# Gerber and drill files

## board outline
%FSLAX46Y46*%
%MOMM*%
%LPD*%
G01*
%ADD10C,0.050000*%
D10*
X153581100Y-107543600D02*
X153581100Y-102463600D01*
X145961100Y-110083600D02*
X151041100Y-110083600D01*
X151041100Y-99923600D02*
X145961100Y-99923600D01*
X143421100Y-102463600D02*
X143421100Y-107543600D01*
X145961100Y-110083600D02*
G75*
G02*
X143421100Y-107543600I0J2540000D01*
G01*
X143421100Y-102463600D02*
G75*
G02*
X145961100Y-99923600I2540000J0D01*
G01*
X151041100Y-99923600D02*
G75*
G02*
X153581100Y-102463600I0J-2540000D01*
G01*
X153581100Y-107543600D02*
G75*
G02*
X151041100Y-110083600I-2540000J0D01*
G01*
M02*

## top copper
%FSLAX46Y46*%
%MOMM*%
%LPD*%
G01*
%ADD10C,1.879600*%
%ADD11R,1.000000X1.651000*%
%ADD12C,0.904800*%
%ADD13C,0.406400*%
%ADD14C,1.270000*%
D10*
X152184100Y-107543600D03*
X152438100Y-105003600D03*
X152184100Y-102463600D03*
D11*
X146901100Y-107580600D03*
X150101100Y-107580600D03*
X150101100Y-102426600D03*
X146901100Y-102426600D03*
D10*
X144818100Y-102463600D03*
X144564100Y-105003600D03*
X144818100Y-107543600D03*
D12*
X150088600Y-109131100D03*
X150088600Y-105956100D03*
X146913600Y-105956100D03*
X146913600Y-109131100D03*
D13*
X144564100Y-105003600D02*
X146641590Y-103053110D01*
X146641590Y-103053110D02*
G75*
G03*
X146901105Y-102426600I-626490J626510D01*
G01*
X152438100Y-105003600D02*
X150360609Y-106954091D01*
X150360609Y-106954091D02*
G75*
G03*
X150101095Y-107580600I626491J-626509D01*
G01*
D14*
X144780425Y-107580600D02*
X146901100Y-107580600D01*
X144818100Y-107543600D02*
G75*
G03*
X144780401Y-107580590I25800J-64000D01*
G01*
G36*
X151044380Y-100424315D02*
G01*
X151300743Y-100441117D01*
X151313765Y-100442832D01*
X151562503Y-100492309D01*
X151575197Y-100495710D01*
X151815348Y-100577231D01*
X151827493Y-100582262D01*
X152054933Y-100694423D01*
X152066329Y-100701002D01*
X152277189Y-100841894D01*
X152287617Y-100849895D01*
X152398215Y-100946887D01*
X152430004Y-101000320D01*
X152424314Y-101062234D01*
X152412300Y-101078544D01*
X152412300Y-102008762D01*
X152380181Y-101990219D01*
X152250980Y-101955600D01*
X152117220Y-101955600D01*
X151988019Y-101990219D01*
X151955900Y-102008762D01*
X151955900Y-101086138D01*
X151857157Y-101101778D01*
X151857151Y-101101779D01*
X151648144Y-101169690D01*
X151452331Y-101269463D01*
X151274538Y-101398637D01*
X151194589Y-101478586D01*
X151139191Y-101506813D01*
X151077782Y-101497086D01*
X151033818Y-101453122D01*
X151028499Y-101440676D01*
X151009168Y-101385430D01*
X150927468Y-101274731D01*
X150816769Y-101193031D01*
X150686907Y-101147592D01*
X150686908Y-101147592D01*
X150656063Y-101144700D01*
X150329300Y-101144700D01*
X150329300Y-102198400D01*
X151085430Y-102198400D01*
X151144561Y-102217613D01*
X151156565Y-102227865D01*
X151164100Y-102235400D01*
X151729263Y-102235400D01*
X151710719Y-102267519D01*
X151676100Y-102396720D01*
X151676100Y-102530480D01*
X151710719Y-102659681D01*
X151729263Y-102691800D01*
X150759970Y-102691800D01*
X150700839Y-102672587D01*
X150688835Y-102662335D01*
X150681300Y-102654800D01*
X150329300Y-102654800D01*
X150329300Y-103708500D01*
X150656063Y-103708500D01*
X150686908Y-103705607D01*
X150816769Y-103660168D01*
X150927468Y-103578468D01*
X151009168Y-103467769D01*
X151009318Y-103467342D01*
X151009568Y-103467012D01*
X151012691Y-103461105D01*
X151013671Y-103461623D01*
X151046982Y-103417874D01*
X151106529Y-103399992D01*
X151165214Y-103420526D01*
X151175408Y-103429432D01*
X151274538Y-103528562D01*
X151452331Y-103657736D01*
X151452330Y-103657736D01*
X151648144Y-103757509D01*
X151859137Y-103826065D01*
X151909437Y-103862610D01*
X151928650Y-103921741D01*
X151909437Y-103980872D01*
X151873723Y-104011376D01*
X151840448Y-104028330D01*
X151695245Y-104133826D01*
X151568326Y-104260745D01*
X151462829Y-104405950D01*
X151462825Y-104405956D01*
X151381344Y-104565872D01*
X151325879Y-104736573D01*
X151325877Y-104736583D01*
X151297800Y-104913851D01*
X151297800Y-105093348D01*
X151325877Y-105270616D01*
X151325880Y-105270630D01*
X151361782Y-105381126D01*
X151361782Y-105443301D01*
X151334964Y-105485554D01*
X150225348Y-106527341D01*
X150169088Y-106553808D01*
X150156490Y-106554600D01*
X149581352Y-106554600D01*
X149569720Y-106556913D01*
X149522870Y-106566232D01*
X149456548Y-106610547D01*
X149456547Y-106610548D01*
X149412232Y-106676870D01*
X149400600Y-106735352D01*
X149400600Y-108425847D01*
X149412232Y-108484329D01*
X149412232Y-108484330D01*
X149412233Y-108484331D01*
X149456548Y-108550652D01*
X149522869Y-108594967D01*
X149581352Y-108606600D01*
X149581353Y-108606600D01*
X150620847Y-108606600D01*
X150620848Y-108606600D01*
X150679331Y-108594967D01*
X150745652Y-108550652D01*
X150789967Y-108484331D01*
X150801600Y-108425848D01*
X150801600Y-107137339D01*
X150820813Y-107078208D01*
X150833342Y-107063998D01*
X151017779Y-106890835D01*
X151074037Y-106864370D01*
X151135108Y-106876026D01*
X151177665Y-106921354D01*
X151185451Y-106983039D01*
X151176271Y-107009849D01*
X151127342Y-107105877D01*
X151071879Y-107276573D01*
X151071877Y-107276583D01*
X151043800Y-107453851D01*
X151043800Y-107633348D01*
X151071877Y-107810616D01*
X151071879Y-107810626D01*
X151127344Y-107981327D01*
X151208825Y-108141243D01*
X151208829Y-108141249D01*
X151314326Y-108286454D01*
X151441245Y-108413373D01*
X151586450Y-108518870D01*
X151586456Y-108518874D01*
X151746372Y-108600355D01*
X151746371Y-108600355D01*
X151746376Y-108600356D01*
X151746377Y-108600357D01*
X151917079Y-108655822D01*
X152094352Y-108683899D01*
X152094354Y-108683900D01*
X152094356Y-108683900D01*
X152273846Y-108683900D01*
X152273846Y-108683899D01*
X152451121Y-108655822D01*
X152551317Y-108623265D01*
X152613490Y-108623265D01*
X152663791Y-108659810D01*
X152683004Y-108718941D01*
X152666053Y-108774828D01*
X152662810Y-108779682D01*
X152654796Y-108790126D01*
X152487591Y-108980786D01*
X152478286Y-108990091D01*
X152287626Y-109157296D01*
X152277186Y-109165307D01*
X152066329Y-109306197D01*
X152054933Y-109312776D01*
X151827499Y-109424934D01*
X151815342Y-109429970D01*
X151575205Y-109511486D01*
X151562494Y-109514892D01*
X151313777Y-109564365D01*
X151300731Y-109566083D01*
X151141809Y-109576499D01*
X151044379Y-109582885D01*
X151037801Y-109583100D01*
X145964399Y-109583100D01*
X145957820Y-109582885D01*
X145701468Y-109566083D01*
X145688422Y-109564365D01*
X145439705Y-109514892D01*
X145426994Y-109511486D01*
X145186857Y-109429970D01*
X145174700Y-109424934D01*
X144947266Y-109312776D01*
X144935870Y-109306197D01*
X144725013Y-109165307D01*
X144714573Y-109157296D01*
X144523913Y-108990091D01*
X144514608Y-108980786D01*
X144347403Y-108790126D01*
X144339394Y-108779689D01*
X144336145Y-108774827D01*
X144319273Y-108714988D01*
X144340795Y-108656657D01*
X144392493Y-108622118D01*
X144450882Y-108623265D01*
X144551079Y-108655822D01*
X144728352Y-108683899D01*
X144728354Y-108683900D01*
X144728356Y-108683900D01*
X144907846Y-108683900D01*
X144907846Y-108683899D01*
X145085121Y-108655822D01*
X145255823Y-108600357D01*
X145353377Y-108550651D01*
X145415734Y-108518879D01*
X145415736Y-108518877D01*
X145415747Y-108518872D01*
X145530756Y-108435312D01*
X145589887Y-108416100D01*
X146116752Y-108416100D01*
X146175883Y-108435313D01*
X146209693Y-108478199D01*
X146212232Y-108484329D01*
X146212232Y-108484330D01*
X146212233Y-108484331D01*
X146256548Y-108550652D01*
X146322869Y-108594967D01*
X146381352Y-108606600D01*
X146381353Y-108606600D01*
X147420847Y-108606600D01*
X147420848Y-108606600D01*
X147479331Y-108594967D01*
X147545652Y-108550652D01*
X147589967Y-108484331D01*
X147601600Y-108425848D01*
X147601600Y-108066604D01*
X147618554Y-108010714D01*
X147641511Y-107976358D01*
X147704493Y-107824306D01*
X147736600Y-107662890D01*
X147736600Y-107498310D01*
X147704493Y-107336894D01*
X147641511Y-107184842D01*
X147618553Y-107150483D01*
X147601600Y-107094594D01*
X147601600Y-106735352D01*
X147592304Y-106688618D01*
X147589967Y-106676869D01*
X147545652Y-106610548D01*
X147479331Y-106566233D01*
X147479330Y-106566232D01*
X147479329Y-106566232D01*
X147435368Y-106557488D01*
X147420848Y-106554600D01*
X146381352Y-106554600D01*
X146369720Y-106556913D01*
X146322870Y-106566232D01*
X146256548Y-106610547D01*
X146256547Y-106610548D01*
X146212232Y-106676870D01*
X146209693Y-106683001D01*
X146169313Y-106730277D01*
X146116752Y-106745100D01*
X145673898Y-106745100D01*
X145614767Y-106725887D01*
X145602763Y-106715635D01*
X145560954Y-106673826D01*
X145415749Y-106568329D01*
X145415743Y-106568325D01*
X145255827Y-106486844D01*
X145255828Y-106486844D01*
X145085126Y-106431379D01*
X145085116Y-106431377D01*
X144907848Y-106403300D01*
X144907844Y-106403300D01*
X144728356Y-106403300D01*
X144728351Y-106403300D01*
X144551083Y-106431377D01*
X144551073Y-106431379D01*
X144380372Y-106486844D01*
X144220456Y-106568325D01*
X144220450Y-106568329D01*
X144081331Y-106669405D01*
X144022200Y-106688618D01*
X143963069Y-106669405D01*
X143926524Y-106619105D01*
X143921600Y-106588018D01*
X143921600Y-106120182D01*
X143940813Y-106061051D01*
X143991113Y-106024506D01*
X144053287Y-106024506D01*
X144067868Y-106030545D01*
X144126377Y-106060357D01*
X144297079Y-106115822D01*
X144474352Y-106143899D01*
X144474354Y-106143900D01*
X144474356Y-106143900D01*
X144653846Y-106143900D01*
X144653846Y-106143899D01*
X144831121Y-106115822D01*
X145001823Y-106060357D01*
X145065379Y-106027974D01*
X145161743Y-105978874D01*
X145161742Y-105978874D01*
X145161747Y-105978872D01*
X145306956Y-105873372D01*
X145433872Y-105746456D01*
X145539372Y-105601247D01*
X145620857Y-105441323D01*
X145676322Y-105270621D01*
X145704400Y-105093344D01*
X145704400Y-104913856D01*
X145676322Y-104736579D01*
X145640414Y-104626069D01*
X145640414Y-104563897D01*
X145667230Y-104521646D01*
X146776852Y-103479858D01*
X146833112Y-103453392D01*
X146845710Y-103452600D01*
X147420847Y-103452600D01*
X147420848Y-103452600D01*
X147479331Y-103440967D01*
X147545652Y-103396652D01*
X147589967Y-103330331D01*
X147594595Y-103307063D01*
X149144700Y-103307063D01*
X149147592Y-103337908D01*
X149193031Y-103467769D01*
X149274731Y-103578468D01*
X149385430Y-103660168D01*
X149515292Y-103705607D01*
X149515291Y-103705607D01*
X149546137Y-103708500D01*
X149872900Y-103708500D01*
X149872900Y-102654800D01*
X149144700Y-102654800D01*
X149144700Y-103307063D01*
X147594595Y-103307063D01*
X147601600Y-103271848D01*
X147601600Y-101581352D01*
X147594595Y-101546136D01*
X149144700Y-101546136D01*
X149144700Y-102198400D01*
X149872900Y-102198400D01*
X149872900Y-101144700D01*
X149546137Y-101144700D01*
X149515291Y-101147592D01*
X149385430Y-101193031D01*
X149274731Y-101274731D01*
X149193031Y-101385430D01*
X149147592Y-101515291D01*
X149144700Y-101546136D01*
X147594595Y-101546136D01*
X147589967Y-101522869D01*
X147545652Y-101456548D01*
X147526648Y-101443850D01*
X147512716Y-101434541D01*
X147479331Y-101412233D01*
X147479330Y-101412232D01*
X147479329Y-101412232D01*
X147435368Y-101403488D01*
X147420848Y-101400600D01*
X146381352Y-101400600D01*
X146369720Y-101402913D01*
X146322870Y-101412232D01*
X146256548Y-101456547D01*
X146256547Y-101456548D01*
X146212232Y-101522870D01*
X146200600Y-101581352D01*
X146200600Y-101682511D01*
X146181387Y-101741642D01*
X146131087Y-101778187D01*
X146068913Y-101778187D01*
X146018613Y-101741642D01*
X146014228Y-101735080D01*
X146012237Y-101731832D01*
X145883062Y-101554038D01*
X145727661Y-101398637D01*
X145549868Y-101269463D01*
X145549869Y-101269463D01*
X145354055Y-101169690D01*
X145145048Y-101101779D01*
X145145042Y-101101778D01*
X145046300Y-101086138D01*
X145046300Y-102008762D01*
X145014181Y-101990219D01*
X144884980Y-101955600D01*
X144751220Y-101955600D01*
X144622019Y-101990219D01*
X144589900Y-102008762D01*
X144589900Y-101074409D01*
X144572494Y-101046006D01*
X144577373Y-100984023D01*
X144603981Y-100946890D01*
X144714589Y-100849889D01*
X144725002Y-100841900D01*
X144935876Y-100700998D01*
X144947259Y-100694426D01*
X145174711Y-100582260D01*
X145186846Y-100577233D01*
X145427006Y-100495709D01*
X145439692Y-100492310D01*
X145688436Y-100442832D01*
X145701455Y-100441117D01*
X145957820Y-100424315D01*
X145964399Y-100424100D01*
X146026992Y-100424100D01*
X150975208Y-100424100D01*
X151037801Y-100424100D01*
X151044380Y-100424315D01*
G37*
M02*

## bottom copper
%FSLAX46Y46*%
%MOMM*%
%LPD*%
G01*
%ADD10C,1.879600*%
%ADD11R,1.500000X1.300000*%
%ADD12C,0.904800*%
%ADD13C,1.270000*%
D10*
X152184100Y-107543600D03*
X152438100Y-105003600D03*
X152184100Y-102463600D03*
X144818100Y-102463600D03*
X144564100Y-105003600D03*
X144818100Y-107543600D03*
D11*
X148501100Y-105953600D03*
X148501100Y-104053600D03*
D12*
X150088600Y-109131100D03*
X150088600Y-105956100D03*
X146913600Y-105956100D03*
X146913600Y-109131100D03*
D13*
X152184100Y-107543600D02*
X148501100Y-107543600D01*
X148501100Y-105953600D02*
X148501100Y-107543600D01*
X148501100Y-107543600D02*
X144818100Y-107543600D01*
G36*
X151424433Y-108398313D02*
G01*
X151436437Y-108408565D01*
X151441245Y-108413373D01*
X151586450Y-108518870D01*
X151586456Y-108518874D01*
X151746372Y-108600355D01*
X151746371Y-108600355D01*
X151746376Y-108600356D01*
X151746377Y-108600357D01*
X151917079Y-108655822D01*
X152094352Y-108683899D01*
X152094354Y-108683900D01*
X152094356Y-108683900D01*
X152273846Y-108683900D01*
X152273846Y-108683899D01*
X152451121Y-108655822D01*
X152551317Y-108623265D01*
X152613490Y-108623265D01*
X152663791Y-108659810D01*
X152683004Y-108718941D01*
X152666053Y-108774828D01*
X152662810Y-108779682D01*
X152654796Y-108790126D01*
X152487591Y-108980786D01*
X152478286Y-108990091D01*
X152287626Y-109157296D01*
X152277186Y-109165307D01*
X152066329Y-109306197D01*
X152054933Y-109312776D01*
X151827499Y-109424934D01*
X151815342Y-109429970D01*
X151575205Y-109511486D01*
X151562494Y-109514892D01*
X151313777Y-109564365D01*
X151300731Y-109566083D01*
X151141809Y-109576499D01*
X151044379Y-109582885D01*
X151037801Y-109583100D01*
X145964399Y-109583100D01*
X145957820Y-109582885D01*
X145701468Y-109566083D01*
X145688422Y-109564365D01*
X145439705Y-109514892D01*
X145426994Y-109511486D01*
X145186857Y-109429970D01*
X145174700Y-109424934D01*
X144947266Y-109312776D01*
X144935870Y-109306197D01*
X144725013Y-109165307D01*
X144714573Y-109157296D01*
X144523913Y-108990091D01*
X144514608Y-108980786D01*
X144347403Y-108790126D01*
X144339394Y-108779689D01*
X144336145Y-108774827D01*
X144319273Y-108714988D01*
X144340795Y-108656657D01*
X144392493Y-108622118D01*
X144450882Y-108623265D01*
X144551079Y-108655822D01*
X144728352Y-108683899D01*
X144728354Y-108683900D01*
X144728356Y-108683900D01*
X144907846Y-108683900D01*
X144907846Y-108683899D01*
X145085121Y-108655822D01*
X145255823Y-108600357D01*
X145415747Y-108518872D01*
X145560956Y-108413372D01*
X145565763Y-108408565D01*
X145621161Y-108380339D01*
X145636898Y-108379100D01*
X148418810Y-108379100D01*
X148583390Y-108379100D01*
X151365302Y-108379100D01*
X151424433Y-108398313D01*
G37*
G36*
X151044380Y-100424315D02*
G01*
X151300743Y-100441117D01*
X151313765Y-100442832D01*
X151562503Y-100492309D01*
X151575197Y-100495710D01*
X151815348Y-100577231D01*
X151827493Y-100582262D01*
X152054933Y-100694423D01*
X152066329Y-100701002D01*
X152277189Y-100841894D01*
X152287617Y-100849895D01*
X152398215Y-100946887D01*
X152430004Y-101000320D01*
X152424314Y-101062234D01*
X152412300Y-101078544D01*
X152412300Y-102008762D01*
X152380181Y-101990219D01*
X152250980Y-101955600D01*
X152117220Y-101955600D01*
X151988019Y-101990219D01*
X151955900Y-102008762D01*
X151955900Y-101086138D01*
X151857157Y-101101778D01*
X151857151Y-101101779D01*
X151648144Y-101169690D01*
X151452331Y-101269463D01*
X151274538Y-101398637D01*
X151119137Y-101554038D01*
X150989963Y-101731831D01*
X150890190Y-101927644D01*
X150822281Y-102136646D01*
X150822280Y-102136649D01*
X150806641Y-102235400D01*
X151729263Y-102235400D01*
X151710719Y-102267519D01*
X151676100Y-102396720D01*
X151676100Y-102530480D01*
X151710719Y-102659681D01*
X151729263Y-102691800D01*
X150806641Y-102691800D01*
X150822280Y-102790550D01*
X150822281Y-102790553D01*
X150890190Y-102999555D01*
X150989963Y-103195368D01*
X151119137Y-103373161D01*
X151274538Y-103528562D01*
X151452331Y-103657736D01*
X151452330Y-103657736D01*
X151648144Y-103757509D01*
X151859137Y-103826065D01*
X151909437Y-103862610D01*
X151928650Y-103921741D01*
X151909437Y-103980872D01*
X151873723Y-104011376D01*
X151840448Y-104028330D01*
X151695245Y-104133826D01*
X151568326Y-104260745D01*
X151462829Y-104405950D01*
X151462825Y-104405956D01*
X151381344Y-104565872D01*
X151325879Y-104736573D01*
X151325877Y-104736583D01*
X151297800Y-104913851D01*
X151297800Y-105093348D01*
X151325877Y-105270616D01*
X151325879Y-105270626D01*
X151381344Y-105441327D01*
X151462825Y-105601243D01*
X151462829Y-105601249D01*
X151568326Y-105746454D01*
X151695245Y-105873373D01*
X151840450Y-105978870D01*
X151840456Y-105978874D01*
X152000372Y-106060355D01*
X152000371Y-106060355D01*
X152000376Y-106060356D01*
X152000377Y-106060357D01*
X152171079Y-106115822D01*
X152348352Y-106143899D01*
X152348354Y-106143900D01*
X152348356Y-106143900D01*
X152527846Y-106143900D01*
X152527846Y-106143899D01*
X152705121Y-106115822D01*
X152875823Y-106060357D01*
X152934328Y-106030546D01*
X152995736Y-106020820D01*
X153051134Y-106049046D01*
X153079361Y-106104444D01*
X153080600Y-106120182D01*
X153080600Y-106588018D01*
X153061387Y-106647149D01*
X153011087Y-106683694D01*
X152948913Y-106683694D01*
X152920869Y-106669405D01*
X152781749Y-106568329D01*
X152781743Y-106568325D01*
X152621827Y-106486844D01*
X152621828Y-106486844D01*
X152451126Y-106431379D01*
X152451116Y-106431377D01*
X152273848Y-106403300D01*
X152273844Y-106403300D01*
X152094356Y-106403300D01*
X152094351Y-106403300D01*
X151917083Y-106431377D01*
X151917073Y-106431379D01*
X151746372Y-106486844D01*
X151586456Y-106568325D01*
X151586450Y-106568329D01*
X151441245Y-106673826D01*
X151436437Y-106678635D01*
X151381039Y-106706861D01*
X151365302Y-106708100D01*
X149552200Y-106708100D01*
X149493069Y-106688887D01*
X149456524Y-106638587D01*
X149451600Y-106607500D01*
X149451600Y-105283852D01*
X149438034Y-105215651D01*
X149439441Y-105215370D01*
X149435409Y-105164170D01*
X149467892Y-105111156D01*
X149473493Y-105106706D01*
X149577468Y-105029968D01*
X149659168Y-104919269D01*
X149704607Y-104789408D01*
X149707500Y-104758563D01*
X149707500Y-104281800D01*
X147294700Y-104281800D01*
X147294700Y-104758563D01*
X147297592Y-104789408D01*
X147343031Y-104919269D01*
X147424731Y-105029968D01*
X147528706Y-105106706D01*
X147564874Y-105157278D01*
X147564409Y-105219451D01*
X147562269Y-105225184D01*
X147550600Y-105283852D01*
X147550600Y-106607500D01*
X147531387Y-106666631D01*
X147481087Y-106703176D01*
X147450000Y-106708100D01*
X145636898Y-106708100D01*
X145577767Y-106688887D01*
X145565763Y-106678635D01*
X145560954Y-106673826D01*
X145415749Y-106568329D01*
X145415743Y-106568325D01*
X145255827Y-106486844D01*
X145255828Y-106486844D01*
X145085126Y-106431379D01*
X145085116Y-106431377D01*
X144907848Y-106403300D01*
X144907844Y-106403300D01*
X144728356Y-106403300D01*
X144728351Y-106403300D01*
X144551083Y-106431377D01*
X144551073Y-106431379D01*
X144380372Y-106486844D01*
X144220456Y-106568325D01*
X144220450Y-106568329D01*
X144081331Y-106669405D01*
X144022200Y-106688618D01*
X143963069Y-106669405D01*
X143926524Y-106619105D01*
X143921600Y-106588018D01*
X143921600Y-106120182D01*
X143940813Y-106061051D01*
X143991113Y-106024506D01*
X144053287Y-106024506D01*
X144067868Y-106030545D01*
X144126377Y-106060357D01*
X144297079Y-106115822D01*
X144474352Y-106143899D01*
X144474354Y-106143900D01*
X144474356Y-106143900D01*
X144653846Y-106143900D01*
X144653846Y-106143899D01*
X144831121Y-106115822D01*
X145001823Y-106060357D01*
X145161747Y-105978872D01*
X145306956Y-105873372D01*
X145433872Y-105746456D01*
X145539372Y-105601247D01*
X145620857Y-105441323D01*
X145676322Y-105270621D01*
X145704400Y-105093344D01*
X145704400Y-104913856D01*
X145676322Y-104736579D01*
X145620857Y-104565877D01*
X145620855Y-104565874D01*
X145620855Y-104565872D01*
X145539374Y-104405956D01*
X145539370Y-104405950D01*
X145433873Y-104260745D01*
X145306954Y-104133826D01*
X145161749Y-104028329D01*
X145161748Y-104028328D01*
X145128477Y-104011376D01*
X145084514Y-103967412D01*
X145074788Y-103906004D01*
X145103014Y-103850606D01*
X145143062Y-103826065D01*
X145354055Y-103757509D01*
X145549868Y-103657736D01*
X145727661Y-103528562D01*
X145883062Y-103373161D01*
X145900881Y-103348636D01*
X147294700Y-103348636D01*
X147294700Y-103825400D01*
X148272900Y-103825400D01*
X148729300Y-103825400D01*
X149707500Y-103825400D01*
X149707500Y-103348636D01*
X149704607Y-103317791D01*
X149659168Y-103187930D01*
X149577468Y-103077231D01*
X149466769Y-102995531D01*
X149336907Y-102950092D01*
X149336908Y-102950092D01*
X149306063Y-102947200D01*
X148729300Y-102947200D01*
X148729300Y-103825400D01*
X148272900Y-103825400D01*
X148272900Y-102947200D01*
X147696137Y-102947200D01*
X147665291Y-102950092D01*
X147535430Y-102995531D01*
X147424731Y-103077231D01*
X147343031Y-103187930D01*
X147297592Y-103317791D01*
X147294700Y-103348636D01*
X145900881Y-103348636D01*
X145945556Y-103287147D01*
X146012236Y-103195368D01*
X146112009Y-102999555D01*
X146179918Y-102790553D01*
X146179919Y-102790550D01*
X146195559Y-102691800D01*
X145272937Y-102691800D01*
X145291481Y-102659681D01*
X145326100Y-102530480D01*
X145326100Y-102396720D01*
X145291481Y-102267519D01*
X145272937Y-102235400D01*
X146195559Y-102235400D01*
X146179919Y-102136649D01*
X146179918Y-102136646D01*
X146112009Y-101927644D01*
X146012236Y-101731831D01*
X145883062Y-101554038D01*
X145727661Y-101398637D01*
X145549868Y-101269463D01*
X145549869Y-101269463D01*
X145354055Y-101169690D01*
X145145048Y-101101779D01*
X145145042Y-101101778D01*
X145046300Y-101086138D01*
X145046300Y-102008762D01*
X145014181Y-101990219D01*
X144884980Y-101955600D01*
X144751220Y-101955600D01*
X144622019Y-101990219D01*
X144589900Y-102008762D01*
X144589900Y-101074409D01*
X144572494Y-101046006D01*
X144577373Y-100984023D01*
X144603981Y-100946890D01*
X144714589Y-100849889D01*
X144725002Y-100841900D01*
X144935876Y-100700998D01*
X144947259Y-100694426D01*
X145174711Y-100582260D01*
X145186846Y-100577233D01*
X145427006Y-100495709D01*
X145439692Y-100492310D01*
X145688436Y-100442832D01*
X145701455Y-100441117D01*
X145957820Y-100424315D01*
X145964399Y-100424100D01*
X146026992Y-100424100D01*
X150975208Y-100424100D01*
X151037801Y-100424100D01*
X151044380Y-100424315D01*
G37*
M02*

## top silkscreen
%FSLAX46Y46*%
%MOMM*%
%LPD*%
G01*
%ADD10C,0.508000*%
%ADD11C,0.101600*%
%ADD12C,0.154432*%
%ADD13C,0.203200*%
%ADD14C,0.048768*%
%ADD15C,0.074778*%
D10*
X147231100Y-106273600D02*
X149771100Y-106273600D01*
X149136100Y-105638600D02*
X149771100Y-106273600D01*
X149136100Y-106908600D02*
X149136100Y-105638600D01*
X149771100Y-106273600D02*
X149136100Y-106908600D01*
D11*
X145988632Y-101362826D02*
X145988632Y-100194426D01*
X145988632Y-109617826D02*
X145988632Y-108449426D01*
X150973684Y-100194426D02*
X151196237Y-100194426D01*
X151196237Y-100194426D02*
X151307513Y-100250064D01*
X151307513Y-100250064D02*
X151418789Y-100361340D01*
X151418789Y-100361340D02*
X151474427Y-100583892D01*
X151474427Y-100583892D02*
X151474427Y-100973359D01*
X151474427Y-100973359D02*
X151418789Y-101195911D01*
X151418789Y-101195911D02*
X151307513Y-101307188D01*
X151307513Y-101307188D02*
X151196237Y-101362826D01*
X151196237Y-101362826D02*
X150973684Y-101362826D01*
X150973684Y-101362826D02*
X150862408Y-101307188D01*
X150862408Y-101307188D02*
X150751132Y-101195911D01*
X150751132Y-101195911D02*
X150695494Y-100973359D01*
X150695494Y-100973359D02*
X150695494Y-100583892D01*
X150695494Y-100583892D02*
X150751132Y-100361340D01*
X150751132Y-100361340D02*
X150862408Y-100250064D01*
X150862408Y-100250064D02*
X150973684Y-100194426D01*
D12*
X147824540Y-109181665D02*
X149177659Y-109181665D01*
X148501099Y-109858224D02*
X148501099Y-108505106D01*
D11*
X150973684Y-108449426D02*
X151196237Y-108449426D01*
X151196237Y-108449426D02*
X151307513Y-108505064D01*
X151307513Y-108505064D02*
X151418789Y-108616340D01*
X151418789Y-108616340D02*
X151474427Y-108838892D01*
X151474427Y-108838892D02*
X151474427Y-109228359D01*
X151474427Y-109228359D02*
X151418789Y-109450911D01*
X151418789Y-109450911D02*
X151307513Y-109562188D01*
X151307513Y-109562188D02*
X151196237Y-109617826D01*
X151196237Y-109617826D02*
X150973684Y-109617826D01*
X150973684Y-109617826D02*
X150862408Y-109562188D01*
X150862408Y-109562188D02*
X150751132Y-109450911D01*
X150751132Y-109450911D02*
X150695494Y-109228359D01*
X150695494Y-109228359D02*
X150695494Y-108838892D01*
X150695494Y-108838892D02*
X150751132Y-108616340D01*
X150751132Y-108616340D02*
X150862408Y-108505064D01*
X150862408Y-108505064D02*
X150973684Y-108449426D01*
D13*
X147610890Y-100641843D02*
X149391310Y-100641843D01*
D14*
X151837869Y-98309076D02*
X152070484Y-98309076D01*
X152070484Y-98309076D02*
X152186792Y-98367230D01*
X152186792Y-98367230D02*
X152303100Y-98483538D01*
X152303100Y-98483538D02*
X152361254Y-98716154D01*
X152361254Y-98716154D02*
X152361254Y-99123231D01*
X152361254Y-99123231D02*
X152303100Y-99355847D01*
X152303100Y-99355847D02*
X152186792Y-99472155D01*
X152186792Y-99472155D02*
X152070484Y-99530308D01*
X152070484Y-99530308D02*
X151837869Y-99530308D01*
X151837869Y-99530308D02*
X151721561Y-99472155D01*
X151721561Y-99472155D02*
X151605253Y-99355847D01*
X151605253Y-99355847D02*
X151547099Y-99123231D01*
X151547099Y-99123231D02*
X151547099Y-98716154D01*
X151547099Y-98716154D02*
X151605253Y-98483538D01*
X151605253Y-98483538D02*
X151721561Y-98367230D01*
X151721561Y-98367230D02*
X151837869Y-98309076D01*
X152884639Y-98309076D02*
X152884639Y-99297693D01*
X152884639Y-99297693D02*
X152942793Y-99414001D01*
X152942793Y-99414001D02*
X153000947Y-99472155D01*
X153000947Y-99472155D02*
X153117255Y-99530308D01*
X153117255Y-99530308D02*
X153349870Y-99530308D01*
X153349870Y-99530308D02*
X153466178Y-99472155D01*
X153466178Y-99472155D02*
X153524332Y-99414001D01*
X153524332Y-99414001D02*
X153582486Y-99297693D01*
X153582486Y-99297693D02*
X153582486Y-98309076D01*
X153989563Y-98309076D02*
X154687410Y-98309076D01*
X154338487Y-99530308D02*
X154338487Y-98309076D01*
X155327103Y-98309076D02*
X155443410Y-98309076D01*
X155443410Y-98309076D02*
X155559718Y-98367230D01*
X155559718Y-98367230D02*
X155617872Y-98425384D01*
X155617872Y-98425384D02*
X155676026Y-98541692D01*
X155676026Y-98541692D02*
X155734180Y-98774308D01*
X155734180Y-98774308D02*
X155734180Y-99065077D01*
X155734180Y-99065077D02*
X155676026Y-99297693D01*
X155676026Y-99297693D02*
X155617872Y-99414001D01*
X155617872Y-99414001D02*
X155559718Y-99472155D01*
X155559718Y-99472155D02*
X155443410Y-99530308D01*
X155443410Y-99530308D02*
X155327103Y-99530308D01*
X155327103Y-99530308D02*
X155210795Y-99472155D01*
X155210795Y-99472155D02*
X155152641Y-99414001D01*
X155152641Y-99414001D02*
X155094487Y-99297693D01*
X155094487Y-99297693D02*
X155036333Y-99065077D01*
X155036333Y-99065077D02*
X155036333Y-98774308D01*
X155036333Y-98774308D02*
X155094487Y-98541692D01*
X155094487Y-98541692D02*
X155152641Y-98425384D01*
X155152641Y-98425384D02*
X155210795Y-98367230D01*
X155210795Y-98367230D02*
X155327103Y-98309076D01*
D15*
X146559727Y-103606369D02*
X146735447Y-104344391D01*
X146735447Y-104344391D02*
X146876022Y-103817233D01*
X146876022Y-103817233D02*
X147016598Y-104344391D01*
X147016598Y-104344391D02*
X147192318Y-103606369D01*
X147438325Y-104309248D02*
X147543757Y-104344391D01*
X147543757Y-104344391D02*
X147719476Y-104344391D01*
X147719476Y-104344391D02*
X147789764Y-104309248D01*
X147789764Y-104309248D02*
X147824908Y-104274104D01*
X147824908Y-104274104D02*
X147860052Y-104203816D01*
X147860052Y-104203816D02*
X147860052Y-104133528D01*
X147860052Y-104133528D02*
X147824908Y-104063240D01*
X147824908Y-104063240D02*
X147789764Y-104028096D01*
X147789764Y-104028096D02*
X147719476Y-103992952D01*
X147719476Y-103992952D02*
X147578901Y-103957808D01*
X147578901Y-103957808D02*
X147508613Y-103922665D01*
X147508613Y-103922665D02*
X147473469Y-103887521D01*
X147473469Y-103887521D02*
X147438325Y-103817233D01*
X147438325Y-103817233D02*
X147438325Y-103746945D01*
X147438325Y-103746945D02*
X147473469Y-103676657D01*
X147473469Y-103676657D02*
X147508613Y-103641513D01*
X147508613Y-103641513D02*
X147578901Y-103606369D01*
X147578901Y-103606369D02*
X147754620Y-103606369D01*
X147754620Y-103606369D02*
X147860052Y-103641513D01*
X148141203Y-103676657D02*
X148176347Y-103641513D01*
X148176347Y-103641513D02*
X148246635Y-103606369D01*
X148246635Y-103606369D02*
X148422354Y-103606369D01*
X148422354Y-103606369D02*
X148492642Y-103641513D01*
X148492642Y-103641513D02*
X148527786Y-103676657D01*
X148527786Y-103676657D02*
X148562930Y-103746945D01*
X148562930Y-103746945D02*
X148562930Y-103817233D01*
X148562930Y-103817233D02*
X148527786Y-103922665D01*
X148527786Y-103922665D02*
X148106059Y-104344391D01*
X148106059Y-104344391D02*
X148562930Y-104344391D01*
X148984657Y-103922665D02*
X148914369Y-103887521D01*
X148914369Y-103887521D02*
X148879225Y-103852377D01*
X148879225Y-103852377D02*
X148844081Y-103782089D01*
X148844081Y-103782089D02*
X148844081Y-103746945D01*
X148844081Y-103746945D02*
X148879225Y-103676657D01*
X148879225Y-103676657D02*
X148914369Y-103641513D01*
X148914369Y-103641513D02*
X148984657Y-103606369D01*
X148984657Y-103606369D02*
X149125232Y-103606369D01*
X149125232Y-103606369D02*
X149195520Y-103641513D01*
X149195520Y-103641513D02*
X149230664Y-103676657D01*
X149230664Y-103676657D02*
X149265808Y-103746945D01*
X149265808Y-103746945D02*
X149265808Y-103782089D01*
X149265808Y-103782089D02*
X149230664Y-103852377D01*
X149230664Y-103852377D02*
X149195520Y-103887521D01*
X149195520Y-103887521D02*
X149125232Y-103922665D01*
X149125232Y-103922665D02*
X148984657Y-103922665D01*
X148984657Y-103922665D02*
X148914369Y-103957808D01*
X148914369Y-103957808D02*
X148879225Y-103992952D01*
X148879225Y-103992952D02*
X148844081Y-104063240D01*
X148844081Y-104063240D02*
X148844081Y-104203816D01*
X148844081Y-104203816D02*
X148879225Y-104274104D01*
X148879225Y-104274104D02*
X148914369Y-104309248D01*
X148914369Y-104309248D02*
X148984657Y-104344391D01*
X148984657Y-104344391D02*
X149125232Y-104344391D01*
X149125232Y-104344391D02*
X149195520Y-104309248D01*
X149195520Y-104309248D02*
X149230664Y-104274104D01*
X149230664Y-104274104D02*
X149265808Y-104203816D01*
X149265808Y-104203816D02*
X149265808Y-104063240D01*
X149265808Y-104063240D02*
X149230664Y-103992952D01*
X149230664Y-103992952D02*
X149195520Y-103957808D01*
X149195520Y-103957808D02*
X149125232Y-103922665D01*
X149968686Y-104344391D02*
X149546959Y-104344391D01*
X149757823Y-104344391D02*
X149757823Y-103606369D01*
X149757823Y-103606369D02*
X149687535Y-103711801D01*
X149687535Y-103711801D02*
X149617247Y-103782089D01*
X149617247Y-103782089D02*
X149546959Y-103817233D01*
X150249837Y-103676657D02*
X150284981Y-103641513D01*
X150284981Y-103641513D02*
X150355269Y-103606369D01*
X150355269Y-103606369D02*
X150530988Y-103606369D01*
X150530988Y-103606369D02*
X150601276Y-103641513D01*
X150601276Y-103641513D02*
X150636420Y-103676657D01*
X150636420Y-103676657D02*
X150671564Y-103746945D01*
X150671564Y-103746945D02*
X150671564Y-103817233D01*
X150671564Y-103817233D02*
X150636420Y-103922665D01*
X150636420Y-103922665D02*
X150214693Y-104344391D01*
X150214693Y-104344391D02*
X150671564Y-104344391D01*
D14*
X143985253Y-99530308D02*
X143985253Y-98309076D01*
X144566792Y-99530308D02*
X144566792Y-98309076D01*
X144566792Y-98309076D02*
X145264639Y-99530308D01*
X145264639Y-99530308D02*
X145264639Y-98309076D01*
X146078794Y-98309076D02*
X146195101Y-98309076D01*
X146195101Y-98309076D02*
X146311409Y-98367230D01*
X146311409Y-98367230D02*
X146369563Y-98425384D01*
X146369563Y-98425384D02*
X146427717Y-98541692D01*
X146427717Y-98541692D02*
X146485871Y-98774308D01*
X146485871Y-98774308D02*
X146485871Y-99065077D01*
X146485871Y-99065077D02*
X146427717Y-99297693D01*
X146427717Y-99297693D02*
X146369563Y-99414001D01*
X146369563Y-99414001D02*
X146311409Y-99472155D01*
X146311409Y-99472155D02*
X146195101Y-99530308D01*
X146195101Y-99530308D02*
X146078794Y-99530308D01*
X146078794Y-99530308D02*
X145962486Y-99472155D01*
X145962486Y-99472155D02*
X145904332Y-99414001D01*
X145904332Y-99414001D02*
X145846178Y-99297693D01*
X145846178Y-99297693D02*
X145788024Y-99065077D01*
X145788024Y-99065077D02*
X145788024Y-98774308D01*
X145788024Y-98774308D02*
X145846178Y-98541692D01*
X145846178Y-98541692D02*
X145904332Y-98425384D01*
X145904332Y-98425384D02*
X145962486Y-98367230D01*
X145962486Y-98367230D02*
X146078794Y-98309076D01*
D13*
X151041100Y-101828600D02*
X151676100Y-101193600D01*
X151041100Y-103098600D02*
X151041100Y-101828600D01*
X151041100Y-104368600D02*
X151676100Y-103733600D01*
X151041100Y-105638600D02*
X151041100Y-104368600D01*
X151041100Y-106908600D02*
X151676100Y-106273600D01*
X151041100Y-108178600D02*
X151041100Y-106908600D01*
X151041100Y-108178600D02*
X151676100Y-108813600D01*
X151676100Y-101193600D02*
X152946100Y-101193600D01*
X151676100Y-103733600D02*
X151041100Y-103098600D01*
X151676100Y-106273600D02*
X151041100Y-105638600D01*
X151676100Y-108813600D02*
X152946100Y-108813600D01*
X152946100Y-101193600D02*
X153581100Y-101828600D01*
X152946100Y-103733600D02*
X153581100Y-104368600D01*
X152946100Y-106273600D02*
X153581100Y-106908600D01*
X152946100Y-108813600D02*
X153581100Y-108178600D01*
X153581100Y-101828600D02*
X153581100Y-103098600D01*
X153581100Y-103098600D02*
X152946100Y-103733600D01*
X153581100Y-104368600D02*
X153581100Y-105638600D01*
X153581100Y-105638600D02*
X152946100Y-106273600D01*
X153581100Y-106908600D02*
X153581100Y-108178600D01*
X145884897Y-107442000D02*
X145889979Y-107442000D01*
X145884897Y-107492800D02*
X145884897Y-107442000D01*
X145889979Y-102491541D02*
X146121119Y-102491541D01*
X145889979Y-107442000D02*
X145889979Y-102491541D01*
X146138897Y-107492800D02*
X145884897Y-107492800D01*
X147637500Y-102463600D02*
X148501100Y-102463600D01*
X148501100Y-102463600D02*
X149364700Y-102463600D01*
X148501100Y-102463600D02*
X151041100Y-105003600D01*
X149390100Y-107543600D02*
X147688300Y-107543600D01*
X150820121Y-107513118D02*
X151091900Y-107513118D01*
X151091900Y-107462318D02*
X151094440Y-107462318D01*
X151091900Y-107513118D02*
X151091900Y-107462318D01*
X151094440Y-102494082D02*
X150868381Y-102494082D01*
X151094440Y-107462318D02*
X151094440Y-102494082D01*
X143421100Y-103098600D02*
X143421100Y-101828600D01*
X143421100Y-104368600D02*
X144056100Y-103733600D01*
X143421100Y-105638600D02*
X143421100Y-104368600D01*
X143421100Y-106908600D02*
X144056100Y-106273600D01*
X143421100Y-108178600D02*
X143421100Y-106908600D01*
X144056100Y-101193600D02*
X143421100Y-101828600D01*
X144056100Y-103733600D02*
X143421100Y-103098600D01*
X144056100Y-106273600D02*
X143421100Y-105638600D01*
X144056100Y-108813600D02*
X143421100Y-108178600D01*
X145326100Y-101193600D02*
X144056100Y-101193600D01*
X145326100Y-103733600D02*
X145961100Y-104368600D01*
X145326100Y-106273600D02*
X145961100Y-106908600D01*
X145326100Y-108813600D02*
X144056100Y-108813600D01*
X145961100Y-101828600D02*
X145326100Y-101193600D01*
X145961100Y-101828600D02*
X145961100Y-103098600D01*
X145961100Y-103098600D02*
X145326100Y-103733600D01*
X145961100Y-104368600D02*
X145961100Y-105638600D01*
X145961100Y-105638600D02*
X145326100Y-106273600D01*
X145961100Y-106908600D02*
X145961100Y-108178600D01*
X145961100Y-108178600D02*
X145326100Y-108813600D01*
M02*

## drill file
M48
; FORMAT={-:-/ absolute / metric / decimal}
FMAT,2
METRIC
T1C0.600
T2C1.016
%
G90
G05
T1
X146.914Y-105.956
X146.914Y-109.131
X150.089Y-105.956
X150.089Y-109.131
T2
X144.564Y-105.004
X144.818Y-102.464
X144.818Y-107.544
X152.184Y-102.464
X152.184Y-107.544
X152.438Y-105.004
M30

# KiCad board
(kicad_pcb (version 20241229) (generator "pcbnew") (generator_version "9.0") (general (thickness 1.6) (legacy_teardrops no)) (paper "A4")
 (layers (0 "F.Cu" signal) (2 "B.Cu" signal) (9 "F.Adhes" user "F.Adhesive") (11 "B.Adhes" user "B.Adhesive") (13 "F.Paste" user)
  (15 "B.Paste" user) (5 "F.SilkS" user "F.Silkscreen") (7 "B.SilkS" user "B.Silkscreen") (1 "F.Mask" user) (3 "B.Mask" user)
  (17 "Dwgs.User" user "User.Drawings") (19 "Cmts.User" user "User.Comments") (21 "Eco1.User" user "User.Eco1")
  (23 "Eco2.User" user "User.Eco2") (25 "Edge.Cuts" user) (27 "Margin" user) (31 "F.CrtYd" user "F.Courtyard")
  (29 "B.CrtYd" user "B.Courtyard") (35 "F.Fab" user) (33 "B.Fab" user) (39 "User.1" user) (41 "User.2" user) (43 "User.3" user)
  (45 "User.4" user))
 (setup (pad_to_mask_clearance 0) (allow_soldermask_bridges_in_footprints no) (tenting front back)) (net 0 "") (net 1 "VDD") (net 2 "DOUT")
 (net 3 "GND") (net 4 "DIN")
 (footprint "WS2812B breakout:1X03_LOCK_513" (layer "F.Cu") (at 152.3111 107.5436 90)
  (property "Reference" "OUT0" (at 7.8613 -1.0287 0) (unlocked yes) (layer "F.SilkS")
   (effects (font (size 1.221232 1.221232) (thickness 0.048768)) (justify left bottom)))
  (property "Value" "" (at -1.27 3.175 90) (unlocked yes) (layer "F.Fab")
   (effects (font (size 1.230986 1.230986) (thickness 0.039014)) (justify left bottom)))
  (fp_line (start 5.715 -1.27) (end 6.35 -0.635) (stroke (width 0.2032) (type solid)) (layer "F.SilkS"))
  (fp_line (start 4.445 -1.27) (end 5.715 -1.27) (stroke (width 0.2032) (type solid)) (layer "F.SilkS"))
  (fp_line (start 3.175 -1.27) (end 3.81 -0.635) (stroke (width 0.2032) (type solid)) (layer "F.SilkS"))
  (fp_line (start 1.905 -1.27) (end 3.175 -1.27) (stroke (width 0.2032) (type solid)) (layer "F.SilkS"))
  (fp_line (start 0.635 -1.27) (end 1.27 -0.635) (stroke (width 0.2032) (type solid)) (layer "F.SilkS"))
  (fp_line (start -0.635 -1.27) (end 0.635 -1.27) (stroke (width 0.2032) (type solid)) (layer "F.SilkS"))
  (fp_line (start -0.635 -1.27) (end -1.27 -0.635) (stroke (width 0.2032) (type solid)) (layer "F.SilkS"))
  (fp_line (start 6.35 -0.635) (end 6.35 0.635) (stroke (width 0.2032) (type solid)) (layer "F.SilkS"))
  (fp_line (start 3.81 -0.635) (end 4.445 -1.27) (stroke (width 0.2032) (type solid)) (layer "F.SilkS"))
  (fp_line (start 1.27 -0.635) (end 1.905 -1.27) (stroke (width 0.2032) (type solid)) (layer "F.SilkS"))
  (fp_line (start -1.27 -0.635) (end -1.27 0.635) (stroke (width 0.2032) (type solid)) (layer "F.SilkS"))
  (fp_line (start 6.35 0.635) (end 5.715 1.27) (stroke (width 0.2032) (type solid)) (layer "F.SilkS"))
  (fp_line (start 3.81 0.635) (end 3.175 1.27) (stroke (width 0.2032) (type solid)) (layer "F.SilkS"))
  (fp_line (start 1.27 0.635) (end 0.635 1.27) (stroke (width 0.2032) (type solid)) (layer "F.SilkS"))
  (fp_line (start -1.27 0.635) (end -0.635 1.27) (stroke (width 0.2032) (type solid)) (layer "F.SilkS"))
  (fp_line (start 5.715 1.27) (end 4.445 1.27) (stroke (width 0.2032) (type solid)) (layer "F.SilkS"))
  (fp_line (start 4.445 1.27) (end 3.81 0.635) (stroke (width 0.2032) (type solid)) (layer "F.SilkS"))
  (fp_line (start 3.175 1.27) (end 1.905 1.27) (stroke (width 0.2032) (type solid)) (layer "F.SilkS"))
  (fp_line (start 1.905 1.27) (end 1.27 0.635) (stroke (width 0.2032) (type solid)) (layer "F.SilkS"))
  (fp_line (start 0.635 1.27) (end -0.635 1.27) (stroke (width 0.2032) (type solid)) (layer "F.SilkS"))
  (pad "1" thru_hole circle (at 0 -0.127 180) (size 1.8796 1.8796) (drill 1.016) (layers "*.Cu" "*.Mask") (remove_unused_layers no)
   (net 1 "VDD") (solder_mask_margin 0.0508) (thermal_bridge_angle 0))
  (pad "2" thru_hole circle (at 2.54 0.127 180) (size 1.8796 1.8796) (drill 1.016) (layers "*.Cu" "*.Mask") (remove_unused_layers no)
   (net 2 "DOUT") (solder_mask_margin 0.0508) (thermal_bridge_angle 0))
  (pad "3" thru_hole circle (at 5.08 -0.127 180) (size 1.8796 1.8796) (drill 1.016) (layers "*.Cu" "*.Mask") (remove_unused_layers no)
   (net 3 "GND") (solder_mask_margin 0.0508) (thermal_bridge_angle 0)))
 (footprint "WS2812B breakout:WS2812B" (layer "F.Cu") (at 148.5011 105.0036 90)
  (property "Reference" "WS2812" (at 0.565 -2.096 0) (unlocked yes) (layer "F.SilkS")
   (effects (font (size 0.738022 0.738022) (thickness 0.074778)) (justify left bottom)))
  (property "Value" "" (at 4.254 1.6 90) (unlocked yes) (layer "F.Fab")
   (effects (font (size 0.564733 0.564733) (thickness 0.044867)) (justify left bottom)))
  (fp_line (start -2.4384 -2.616203) (end -2.4384 -2.611121) (stroke (width 0.2032) (type solid)) (layer "F.SilkS"))
  (fp_line (start -2.4892 -2.616203) (end -2.4384 -2.616203) (stroke (width 0.2032) (type solid)) (layer "F.SilkS"))
  (fp_line (start 2.512059 -2.611121) (end 2.512059 -2.379981) (stroke (width 0.2032) (type solid)) (layer "F.SilkS"))
  (fp_line (start -2.4384 -2.611121) (end 2.512059 -2.611121) (stroke (width 0.2032) (type solid)) (layer "F.SilkS"))
  (fp_line (start -2.4892 -2.362203) (end -2.4892 -2.616203) (stroke (width 0.2032) (type solid)) (layer "F.SilkS"))
  (fp_line (start 2.54 -0.8636) (end 2.54 0) (stroke (width 0.2032) (type solid)) (layer "F.SilkS"))
  (fp_line (start 2.54 0) (end 2.54 0.8636) (stroke (width 0.2032) (type solid)) (layer "F.SilkS"))
  (fp_line (start 2.54 0) (end 0 2.54) (stroke (width 0.2032) (type solid)) (layer "F.SilkS"))
  (fp_line (start -2.54 0.889) (end -2.54 -0.8128) (stroke (width 0.2032) (type solid)) (layer "F.SilkS"))
  (fp_line (start -2.509518 2.319021) (end -2.509518 2.5908) (stroke (width 0.2032) (type solid)) (layer "F.SilkS"))
  (fp_line (start -2.458718 2.5908) (end -2.458718 2.59334) (stroke (width 0.2032) (type solid)) (layer "F.SilkS"))
  (fp_line (start -2.509518 2.5908) (end -2.458718 2.5908) (stroke (width 0.2032) (type solid)) (layer "F.SilkS"))
  (fp_line (start 2.509518 2.59334) (end 2.509518 2.367281) (stroke (width 0.2032) (type solid)) (layer "F.SilkS"))
  (fp_line (start -2.458718 2.59334) (end 2.509518 2.59334) (stroke (width 0.2032) (type solid)) (layer "F.SilkS"))
  (pad "1" smd rect (at -2.577 -1.6 90) (size 1.651 1) (layers "F.Cu" "F.Mask" "F.Paste") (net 1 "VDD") (solder_mask_margin 0.0508)
   (solder_paste_margin 0) (thermal_bridge_angle 0))
  (pad "2" smd rect (at -2.577 1.6 90) (size 1.651 1) (layers "F.Cu" "F.Mask" "F.Paste") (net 2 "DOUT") (solder_mask_margin 0.0508)
   (solder_paste_margin 0) (thermal_bridge_angle 0))
  (pad "3" smd rect (at 2.577 1.6 90) (size 1.651 1) (layers "F.Cu" "F.Mask" "F.Paste") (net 3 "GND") (solder_mask_margin 0.0508)
   (solder_paste_margin 0) (thermal_bridge_angle 0))
  (pad "4" smd rect (at 2.577 -1.6 90) (size 1.651 1) (layers "F.Cu" "F.Mask" "F.Paste") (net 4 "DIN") (solder_mask_margin 0.0508)
   (solder_paste_margin 0) (thermal_bridge_angle 0)))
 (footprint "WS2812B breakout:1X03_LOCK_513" (layer "F.Cu") (at 144.6911 102.4636 -90)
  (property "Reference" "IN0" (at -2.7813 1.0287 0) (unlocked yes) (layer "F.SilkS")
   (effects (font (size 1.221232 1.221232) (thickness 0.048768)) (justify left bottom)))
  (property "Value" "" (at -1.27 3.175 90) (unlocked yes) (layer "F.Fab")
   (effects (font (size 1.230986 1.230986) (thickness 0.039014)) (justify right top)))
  (fp_line (start 0.635 1.27) (end -0.635 1.27) (stroke (width 0.2032) (type solid)) (layer "F.SilkS"))
  (fp_line (start 1.905 1.27) (end 1.27 0.635) (stroke (width 0.2032) (type solid)) (layer "F.SilkS"))
  (fp_line (start 3.175 1.27) (end 1.905 1.27) (stroke (width 0.2032) (type solid)) (layer "F.SilkS"))
  (fp_line (start 4.445 1.27) (end 3.81 0.635) (stroke (width 0.2032) (type solid)) (layer "F.SilkS"))
  (fp_line (start 5.715 1.27) (end 4.445 1.27) (stroke (width 0.2032) (type solid)) (layer "F.SilkS"))
  (fp_line (start -1.27 0.635) (end -0.635 1.27) (stroke (width 0.2032) (type solid)) (layer "F.SilkS"))
  (fp_line (start 1.27 0.635) (end 0.635 1.27) (stroke (width 0.2032) (type solid)) (layer "F.SilkS"))
  (fp_line (start 3.81 0.635) (end 3.175 1.27) (stroke (width 0.2032) (type solid)) (layer "F.SilkS"))
  (fp_line (start 6.35 0.635) (end 5.715 1.27) (stroke (width 0.2032) (type solid)) (layer "F.SilkS"))
  (fp_line (start -1.27 -0.635) (end -1.27 0.635) (stroke (width 0.2032) (type solid)) (layer "F.SilkS"))
  (fp_line (start 1.27 -0.635) (end 1.905 -1.27) (stroke (width 0.2032) (type solid)) (layer "F.SilkS"))
  (fp_line (start 3.81 -0.635) (end 4.445 -1.27) (stroke (width 0.2032) (type solid)) (layer "F.SilkS"))
  (fp_line (start 6.35 -0.635) (end 6.35 0.635) (stroke (width 0.2032) (type solid)) (layer "F.SilkS"))
  (fp_line (start -0.635 -1.27) (end -1.27 -0.635) (stroke (width 0.2032) (type solid)) (layer "F.SilkS"))
  (fp_line (start -0.635 -1.27) (end 0.635 -1.27) (stroke (width 0.2032) (type solid)) (layer "F.SilkS"))
  (fp_line (start 0.635 -1.27) (end 1.27 -0.635) (stroke (width 0.2032) (type solid)) (layer "F.SilkS"))
  (fp_line (start 1.905 -1.27) (end 3.175 -1.27) (stroke (width 0.2032) (type solid)) (layer "F.SilkS"))
  (fp_line (start 3.175 -1.27) (end 3.81 -0.635) (stroke (width 0.2032) (type solid)) (layer "F.SilkS"))
  (fp_line (start 4.445 -1.27) (end 5.715 -1.27) (stroke (width 0.2032) (type solid)) (layer "F.SilkS"))
  (fp_line (start 5.715 -1.27) (end 6.35 -0.635) (stroke (width 0.2032) (type solid)) (layer "F.SilkS"))
  (pad "1" thru_hole circle (at 0 -0.127) (size 1.8796 1.8796) (drill 1.016) (layers "*.Cu" "*.Mask") (remove_unused_layers no)
   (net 3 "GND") (solder_mask_margin 0.0508) (thermal_bridge_angle 0))
  (pad "2" thru_hole circle (at 2.54 0.127) (size 1.8796 1.8796) (drill 1.016) (layers "*.Cu" "*.Mask") (remove_unused_layers no)
   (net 4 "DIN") (solder_mask_margin 0.0508) (thermal_bridge_angle 0))
  (pad "3" thru_hole circle (at 5.08 -0.127) (size 1.8796 1.8796) (drill 1.016) (layers "*.Cu" "*.Mask") (remove_unused_layers no)
   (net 1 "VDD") (solder_mask_margin 0.0508) (thermal_bridge_angle 0)))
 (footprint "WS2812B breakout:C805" (layer "B.Cu") (at 148.5011 105.0036 90)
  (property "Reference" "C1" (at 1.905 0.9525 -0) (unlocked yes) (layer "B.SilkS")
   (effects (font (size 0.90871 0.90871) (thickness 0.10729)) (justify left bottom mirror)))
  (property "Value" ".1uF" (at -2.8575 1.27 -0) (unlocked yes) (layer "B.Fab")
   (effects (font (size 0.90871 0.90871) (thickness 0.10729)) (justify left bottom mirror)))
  (pad "1" smd rect (at -0.95 0 90) (size 1.3 1.5) (layers "B.Cu" "B.Mask" "B.Paste") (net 1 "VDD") (solder_mask_margin 0.0508)
   (solder_paste_margin 0) (thermal_bridge_angle 0))
  (pad "2" smd rect (at 0.95 0 90) (size 1.3 1.5) (layers "B.Cu" "B.Mask" "B.Paste") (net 3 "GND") (solder_mask_margin 0.0508)
   (solder_paste_margin 0) (thermal_bridge_angle 0)))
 (gr_line (start 147.2311 106.2736) (end 149.7711 106.2736) (stroke (width 0.508) (type solid)) (layer "F.SilkS"))
 (gr_line (start 149.1361 105.6386) (end 149.7711 106.2736) (stroke (width 0.508) (type solid)) (layer "F.SilkS"))
 (gr_line (start 149.1361 106.9086) (end 149.1361 105.6386) (stroke (width 0.508) (type solid)) (layer "F.SilkS"))
 (gr_line (start 149.7711 106.2736) (end 149.1361 106.9086) (stroke (width 0.508) (type solid)) (layer "F.SilkS"))
 (gr_line (start 153.5811 107.5436) (end 153.5811 102.4636) (stroke (width 0.05) (type solid)) (layer "Edge.Cuts"))
 (gr_line (start 145.9611 110.0836) (end 151.0411 110.0836) (stroke (width 0.05) (type solid)) (layer "Edge.Cuts"))
 (gr_line (start 151.0411 99.9236) (end 145.9611 99.9236) (stroke (width 0.05) (type solid)) (layer "Edge.Cuts"))
 (gr_line (start 143.4211 102.4636) (end 143.4211 107.5436) (stroke (width 0.05) (type solid)) (layer "Edge.Cuts"))
 (gr_arc (start 145.9611 110.0836) (mid 144.165049 109.339651) (end 143.4211 107.5436) (stroke (width 0.05) (type solid))
  (layer "Edge.Cuts"))
 (gr_arc (start 143.4211 102.4636) (mid 144.165049 100.667549) (end 145.9611 99.9236) (stroke (width 0.05) (type solid)) (layer "Edge.Cuts"))
 (gr_arc (start 151.0411 99.9236) (mid 152.837151 100.667549) (end 153.5811 102.4636) (stroke (width 0.05) (type solid)) (layer "Edge.Cuts"))
 (gr_arc (start 153.5811 107.5436) (mid 152.837151 109.339651) (end 151.0411 110.0836) (stroke (width 0.05) (type solid))
  (layer "Edge.Cuts"))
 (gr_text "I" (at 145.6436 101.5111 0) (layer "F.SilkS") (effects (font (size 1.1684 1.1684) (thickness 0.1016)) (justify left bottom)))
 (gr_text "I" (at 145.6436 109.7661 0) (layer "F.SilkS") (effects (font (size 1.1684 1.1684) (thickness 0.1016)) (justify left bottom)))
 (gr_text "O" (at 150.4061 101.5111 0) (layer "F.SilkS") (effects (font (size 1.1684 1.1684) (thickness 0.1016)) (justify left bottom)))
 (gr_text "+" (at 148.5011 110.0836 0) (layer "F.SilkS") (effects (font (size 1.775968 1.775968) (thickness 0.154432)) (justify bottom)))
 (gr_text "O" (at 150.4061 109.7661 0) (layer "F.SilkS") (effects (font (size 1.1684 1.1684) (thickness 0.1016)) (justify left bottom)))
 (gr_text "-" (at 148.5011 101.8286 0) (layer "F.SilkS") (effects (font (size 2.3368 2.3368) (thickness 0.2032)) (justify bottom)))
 (segment (start 144.5641 105.0036) (end 146.64159 103.05311) (width 0.4064) (layer "F.Cu") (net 4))
 (arc (start 146.64159 103.05311) (mid 146.833655 102.765665) (end 146.9011 102.4266) (width 0.4064) (layer "F.Cu") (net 4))
 (segment (start 152.4381 105.0036) (end 150.360609 106.954091) (width 0.4064) (layer "F.Cu") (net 2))
 (arc (start 150.360609 106.954091) (mid 150.168544 107.241536) (end 150.1011 107.5806) (width 0.4064) (layer "F.Cu") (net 2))
 (segment (start 144.780425 107.5806) (end 146.9011 107.5806) (width 1.27) (layer "F.Cu") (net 1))
 (arc (start 144.8181 107.5436) (mid 144.795582 107.558353) (end 144.780425 107.5806) (width 1.27) (layer "F.Cu") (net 1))
 (segment (start 152.1841 107.5436) (end 148.5011 107.5436) (width 1.27) (layer "B.Cu") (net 1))
 (segment (start 148.5011 105.9536) (end 148.5011 107.5436) (width 1.27) (layer "B.Cu") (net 1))
 (segment (start 148.5011 107.5436) (end 144.8181 107.5436) (width 1.27) (layer "B.Cu") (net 1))
 (via (at 150.0886 109.1311) (size 0.9048) (drill 0.6) (layers "F.Cu" "B.Cu") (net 3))
 (via (at 150.0886 105.9561) (size 0.9048) (drill 0.6) (layers "F.Cu" "B.Cu") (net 3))
 (via (at 146.9136 105.9561) (size 0.9048) (drill 0.6) (layers "F.Cu" "B.Cu") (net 3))
 (via (at 146.9136 109.1311) (size 0.9048) (drill 0.6) (layers "F.Cu" "B.Cu") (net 3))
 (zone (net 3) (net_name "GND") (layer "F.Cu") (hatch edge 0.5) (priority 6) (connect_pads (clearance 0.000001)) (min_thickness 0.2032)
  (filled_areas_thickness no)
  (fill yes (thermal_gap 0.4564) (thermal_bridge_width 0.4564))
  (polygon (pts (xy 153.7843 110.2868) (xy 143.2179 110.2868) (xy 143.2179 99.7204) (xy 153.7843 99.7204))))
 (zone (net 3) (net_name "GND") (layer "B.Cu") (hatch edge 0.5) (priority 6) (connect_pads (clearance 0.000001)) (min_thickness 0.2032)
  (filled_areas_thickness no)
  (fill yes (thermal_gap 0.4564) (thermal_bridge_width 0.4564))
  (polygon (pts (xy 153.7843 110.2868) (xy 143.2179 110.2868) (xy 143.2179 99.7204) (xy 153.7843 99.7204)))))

